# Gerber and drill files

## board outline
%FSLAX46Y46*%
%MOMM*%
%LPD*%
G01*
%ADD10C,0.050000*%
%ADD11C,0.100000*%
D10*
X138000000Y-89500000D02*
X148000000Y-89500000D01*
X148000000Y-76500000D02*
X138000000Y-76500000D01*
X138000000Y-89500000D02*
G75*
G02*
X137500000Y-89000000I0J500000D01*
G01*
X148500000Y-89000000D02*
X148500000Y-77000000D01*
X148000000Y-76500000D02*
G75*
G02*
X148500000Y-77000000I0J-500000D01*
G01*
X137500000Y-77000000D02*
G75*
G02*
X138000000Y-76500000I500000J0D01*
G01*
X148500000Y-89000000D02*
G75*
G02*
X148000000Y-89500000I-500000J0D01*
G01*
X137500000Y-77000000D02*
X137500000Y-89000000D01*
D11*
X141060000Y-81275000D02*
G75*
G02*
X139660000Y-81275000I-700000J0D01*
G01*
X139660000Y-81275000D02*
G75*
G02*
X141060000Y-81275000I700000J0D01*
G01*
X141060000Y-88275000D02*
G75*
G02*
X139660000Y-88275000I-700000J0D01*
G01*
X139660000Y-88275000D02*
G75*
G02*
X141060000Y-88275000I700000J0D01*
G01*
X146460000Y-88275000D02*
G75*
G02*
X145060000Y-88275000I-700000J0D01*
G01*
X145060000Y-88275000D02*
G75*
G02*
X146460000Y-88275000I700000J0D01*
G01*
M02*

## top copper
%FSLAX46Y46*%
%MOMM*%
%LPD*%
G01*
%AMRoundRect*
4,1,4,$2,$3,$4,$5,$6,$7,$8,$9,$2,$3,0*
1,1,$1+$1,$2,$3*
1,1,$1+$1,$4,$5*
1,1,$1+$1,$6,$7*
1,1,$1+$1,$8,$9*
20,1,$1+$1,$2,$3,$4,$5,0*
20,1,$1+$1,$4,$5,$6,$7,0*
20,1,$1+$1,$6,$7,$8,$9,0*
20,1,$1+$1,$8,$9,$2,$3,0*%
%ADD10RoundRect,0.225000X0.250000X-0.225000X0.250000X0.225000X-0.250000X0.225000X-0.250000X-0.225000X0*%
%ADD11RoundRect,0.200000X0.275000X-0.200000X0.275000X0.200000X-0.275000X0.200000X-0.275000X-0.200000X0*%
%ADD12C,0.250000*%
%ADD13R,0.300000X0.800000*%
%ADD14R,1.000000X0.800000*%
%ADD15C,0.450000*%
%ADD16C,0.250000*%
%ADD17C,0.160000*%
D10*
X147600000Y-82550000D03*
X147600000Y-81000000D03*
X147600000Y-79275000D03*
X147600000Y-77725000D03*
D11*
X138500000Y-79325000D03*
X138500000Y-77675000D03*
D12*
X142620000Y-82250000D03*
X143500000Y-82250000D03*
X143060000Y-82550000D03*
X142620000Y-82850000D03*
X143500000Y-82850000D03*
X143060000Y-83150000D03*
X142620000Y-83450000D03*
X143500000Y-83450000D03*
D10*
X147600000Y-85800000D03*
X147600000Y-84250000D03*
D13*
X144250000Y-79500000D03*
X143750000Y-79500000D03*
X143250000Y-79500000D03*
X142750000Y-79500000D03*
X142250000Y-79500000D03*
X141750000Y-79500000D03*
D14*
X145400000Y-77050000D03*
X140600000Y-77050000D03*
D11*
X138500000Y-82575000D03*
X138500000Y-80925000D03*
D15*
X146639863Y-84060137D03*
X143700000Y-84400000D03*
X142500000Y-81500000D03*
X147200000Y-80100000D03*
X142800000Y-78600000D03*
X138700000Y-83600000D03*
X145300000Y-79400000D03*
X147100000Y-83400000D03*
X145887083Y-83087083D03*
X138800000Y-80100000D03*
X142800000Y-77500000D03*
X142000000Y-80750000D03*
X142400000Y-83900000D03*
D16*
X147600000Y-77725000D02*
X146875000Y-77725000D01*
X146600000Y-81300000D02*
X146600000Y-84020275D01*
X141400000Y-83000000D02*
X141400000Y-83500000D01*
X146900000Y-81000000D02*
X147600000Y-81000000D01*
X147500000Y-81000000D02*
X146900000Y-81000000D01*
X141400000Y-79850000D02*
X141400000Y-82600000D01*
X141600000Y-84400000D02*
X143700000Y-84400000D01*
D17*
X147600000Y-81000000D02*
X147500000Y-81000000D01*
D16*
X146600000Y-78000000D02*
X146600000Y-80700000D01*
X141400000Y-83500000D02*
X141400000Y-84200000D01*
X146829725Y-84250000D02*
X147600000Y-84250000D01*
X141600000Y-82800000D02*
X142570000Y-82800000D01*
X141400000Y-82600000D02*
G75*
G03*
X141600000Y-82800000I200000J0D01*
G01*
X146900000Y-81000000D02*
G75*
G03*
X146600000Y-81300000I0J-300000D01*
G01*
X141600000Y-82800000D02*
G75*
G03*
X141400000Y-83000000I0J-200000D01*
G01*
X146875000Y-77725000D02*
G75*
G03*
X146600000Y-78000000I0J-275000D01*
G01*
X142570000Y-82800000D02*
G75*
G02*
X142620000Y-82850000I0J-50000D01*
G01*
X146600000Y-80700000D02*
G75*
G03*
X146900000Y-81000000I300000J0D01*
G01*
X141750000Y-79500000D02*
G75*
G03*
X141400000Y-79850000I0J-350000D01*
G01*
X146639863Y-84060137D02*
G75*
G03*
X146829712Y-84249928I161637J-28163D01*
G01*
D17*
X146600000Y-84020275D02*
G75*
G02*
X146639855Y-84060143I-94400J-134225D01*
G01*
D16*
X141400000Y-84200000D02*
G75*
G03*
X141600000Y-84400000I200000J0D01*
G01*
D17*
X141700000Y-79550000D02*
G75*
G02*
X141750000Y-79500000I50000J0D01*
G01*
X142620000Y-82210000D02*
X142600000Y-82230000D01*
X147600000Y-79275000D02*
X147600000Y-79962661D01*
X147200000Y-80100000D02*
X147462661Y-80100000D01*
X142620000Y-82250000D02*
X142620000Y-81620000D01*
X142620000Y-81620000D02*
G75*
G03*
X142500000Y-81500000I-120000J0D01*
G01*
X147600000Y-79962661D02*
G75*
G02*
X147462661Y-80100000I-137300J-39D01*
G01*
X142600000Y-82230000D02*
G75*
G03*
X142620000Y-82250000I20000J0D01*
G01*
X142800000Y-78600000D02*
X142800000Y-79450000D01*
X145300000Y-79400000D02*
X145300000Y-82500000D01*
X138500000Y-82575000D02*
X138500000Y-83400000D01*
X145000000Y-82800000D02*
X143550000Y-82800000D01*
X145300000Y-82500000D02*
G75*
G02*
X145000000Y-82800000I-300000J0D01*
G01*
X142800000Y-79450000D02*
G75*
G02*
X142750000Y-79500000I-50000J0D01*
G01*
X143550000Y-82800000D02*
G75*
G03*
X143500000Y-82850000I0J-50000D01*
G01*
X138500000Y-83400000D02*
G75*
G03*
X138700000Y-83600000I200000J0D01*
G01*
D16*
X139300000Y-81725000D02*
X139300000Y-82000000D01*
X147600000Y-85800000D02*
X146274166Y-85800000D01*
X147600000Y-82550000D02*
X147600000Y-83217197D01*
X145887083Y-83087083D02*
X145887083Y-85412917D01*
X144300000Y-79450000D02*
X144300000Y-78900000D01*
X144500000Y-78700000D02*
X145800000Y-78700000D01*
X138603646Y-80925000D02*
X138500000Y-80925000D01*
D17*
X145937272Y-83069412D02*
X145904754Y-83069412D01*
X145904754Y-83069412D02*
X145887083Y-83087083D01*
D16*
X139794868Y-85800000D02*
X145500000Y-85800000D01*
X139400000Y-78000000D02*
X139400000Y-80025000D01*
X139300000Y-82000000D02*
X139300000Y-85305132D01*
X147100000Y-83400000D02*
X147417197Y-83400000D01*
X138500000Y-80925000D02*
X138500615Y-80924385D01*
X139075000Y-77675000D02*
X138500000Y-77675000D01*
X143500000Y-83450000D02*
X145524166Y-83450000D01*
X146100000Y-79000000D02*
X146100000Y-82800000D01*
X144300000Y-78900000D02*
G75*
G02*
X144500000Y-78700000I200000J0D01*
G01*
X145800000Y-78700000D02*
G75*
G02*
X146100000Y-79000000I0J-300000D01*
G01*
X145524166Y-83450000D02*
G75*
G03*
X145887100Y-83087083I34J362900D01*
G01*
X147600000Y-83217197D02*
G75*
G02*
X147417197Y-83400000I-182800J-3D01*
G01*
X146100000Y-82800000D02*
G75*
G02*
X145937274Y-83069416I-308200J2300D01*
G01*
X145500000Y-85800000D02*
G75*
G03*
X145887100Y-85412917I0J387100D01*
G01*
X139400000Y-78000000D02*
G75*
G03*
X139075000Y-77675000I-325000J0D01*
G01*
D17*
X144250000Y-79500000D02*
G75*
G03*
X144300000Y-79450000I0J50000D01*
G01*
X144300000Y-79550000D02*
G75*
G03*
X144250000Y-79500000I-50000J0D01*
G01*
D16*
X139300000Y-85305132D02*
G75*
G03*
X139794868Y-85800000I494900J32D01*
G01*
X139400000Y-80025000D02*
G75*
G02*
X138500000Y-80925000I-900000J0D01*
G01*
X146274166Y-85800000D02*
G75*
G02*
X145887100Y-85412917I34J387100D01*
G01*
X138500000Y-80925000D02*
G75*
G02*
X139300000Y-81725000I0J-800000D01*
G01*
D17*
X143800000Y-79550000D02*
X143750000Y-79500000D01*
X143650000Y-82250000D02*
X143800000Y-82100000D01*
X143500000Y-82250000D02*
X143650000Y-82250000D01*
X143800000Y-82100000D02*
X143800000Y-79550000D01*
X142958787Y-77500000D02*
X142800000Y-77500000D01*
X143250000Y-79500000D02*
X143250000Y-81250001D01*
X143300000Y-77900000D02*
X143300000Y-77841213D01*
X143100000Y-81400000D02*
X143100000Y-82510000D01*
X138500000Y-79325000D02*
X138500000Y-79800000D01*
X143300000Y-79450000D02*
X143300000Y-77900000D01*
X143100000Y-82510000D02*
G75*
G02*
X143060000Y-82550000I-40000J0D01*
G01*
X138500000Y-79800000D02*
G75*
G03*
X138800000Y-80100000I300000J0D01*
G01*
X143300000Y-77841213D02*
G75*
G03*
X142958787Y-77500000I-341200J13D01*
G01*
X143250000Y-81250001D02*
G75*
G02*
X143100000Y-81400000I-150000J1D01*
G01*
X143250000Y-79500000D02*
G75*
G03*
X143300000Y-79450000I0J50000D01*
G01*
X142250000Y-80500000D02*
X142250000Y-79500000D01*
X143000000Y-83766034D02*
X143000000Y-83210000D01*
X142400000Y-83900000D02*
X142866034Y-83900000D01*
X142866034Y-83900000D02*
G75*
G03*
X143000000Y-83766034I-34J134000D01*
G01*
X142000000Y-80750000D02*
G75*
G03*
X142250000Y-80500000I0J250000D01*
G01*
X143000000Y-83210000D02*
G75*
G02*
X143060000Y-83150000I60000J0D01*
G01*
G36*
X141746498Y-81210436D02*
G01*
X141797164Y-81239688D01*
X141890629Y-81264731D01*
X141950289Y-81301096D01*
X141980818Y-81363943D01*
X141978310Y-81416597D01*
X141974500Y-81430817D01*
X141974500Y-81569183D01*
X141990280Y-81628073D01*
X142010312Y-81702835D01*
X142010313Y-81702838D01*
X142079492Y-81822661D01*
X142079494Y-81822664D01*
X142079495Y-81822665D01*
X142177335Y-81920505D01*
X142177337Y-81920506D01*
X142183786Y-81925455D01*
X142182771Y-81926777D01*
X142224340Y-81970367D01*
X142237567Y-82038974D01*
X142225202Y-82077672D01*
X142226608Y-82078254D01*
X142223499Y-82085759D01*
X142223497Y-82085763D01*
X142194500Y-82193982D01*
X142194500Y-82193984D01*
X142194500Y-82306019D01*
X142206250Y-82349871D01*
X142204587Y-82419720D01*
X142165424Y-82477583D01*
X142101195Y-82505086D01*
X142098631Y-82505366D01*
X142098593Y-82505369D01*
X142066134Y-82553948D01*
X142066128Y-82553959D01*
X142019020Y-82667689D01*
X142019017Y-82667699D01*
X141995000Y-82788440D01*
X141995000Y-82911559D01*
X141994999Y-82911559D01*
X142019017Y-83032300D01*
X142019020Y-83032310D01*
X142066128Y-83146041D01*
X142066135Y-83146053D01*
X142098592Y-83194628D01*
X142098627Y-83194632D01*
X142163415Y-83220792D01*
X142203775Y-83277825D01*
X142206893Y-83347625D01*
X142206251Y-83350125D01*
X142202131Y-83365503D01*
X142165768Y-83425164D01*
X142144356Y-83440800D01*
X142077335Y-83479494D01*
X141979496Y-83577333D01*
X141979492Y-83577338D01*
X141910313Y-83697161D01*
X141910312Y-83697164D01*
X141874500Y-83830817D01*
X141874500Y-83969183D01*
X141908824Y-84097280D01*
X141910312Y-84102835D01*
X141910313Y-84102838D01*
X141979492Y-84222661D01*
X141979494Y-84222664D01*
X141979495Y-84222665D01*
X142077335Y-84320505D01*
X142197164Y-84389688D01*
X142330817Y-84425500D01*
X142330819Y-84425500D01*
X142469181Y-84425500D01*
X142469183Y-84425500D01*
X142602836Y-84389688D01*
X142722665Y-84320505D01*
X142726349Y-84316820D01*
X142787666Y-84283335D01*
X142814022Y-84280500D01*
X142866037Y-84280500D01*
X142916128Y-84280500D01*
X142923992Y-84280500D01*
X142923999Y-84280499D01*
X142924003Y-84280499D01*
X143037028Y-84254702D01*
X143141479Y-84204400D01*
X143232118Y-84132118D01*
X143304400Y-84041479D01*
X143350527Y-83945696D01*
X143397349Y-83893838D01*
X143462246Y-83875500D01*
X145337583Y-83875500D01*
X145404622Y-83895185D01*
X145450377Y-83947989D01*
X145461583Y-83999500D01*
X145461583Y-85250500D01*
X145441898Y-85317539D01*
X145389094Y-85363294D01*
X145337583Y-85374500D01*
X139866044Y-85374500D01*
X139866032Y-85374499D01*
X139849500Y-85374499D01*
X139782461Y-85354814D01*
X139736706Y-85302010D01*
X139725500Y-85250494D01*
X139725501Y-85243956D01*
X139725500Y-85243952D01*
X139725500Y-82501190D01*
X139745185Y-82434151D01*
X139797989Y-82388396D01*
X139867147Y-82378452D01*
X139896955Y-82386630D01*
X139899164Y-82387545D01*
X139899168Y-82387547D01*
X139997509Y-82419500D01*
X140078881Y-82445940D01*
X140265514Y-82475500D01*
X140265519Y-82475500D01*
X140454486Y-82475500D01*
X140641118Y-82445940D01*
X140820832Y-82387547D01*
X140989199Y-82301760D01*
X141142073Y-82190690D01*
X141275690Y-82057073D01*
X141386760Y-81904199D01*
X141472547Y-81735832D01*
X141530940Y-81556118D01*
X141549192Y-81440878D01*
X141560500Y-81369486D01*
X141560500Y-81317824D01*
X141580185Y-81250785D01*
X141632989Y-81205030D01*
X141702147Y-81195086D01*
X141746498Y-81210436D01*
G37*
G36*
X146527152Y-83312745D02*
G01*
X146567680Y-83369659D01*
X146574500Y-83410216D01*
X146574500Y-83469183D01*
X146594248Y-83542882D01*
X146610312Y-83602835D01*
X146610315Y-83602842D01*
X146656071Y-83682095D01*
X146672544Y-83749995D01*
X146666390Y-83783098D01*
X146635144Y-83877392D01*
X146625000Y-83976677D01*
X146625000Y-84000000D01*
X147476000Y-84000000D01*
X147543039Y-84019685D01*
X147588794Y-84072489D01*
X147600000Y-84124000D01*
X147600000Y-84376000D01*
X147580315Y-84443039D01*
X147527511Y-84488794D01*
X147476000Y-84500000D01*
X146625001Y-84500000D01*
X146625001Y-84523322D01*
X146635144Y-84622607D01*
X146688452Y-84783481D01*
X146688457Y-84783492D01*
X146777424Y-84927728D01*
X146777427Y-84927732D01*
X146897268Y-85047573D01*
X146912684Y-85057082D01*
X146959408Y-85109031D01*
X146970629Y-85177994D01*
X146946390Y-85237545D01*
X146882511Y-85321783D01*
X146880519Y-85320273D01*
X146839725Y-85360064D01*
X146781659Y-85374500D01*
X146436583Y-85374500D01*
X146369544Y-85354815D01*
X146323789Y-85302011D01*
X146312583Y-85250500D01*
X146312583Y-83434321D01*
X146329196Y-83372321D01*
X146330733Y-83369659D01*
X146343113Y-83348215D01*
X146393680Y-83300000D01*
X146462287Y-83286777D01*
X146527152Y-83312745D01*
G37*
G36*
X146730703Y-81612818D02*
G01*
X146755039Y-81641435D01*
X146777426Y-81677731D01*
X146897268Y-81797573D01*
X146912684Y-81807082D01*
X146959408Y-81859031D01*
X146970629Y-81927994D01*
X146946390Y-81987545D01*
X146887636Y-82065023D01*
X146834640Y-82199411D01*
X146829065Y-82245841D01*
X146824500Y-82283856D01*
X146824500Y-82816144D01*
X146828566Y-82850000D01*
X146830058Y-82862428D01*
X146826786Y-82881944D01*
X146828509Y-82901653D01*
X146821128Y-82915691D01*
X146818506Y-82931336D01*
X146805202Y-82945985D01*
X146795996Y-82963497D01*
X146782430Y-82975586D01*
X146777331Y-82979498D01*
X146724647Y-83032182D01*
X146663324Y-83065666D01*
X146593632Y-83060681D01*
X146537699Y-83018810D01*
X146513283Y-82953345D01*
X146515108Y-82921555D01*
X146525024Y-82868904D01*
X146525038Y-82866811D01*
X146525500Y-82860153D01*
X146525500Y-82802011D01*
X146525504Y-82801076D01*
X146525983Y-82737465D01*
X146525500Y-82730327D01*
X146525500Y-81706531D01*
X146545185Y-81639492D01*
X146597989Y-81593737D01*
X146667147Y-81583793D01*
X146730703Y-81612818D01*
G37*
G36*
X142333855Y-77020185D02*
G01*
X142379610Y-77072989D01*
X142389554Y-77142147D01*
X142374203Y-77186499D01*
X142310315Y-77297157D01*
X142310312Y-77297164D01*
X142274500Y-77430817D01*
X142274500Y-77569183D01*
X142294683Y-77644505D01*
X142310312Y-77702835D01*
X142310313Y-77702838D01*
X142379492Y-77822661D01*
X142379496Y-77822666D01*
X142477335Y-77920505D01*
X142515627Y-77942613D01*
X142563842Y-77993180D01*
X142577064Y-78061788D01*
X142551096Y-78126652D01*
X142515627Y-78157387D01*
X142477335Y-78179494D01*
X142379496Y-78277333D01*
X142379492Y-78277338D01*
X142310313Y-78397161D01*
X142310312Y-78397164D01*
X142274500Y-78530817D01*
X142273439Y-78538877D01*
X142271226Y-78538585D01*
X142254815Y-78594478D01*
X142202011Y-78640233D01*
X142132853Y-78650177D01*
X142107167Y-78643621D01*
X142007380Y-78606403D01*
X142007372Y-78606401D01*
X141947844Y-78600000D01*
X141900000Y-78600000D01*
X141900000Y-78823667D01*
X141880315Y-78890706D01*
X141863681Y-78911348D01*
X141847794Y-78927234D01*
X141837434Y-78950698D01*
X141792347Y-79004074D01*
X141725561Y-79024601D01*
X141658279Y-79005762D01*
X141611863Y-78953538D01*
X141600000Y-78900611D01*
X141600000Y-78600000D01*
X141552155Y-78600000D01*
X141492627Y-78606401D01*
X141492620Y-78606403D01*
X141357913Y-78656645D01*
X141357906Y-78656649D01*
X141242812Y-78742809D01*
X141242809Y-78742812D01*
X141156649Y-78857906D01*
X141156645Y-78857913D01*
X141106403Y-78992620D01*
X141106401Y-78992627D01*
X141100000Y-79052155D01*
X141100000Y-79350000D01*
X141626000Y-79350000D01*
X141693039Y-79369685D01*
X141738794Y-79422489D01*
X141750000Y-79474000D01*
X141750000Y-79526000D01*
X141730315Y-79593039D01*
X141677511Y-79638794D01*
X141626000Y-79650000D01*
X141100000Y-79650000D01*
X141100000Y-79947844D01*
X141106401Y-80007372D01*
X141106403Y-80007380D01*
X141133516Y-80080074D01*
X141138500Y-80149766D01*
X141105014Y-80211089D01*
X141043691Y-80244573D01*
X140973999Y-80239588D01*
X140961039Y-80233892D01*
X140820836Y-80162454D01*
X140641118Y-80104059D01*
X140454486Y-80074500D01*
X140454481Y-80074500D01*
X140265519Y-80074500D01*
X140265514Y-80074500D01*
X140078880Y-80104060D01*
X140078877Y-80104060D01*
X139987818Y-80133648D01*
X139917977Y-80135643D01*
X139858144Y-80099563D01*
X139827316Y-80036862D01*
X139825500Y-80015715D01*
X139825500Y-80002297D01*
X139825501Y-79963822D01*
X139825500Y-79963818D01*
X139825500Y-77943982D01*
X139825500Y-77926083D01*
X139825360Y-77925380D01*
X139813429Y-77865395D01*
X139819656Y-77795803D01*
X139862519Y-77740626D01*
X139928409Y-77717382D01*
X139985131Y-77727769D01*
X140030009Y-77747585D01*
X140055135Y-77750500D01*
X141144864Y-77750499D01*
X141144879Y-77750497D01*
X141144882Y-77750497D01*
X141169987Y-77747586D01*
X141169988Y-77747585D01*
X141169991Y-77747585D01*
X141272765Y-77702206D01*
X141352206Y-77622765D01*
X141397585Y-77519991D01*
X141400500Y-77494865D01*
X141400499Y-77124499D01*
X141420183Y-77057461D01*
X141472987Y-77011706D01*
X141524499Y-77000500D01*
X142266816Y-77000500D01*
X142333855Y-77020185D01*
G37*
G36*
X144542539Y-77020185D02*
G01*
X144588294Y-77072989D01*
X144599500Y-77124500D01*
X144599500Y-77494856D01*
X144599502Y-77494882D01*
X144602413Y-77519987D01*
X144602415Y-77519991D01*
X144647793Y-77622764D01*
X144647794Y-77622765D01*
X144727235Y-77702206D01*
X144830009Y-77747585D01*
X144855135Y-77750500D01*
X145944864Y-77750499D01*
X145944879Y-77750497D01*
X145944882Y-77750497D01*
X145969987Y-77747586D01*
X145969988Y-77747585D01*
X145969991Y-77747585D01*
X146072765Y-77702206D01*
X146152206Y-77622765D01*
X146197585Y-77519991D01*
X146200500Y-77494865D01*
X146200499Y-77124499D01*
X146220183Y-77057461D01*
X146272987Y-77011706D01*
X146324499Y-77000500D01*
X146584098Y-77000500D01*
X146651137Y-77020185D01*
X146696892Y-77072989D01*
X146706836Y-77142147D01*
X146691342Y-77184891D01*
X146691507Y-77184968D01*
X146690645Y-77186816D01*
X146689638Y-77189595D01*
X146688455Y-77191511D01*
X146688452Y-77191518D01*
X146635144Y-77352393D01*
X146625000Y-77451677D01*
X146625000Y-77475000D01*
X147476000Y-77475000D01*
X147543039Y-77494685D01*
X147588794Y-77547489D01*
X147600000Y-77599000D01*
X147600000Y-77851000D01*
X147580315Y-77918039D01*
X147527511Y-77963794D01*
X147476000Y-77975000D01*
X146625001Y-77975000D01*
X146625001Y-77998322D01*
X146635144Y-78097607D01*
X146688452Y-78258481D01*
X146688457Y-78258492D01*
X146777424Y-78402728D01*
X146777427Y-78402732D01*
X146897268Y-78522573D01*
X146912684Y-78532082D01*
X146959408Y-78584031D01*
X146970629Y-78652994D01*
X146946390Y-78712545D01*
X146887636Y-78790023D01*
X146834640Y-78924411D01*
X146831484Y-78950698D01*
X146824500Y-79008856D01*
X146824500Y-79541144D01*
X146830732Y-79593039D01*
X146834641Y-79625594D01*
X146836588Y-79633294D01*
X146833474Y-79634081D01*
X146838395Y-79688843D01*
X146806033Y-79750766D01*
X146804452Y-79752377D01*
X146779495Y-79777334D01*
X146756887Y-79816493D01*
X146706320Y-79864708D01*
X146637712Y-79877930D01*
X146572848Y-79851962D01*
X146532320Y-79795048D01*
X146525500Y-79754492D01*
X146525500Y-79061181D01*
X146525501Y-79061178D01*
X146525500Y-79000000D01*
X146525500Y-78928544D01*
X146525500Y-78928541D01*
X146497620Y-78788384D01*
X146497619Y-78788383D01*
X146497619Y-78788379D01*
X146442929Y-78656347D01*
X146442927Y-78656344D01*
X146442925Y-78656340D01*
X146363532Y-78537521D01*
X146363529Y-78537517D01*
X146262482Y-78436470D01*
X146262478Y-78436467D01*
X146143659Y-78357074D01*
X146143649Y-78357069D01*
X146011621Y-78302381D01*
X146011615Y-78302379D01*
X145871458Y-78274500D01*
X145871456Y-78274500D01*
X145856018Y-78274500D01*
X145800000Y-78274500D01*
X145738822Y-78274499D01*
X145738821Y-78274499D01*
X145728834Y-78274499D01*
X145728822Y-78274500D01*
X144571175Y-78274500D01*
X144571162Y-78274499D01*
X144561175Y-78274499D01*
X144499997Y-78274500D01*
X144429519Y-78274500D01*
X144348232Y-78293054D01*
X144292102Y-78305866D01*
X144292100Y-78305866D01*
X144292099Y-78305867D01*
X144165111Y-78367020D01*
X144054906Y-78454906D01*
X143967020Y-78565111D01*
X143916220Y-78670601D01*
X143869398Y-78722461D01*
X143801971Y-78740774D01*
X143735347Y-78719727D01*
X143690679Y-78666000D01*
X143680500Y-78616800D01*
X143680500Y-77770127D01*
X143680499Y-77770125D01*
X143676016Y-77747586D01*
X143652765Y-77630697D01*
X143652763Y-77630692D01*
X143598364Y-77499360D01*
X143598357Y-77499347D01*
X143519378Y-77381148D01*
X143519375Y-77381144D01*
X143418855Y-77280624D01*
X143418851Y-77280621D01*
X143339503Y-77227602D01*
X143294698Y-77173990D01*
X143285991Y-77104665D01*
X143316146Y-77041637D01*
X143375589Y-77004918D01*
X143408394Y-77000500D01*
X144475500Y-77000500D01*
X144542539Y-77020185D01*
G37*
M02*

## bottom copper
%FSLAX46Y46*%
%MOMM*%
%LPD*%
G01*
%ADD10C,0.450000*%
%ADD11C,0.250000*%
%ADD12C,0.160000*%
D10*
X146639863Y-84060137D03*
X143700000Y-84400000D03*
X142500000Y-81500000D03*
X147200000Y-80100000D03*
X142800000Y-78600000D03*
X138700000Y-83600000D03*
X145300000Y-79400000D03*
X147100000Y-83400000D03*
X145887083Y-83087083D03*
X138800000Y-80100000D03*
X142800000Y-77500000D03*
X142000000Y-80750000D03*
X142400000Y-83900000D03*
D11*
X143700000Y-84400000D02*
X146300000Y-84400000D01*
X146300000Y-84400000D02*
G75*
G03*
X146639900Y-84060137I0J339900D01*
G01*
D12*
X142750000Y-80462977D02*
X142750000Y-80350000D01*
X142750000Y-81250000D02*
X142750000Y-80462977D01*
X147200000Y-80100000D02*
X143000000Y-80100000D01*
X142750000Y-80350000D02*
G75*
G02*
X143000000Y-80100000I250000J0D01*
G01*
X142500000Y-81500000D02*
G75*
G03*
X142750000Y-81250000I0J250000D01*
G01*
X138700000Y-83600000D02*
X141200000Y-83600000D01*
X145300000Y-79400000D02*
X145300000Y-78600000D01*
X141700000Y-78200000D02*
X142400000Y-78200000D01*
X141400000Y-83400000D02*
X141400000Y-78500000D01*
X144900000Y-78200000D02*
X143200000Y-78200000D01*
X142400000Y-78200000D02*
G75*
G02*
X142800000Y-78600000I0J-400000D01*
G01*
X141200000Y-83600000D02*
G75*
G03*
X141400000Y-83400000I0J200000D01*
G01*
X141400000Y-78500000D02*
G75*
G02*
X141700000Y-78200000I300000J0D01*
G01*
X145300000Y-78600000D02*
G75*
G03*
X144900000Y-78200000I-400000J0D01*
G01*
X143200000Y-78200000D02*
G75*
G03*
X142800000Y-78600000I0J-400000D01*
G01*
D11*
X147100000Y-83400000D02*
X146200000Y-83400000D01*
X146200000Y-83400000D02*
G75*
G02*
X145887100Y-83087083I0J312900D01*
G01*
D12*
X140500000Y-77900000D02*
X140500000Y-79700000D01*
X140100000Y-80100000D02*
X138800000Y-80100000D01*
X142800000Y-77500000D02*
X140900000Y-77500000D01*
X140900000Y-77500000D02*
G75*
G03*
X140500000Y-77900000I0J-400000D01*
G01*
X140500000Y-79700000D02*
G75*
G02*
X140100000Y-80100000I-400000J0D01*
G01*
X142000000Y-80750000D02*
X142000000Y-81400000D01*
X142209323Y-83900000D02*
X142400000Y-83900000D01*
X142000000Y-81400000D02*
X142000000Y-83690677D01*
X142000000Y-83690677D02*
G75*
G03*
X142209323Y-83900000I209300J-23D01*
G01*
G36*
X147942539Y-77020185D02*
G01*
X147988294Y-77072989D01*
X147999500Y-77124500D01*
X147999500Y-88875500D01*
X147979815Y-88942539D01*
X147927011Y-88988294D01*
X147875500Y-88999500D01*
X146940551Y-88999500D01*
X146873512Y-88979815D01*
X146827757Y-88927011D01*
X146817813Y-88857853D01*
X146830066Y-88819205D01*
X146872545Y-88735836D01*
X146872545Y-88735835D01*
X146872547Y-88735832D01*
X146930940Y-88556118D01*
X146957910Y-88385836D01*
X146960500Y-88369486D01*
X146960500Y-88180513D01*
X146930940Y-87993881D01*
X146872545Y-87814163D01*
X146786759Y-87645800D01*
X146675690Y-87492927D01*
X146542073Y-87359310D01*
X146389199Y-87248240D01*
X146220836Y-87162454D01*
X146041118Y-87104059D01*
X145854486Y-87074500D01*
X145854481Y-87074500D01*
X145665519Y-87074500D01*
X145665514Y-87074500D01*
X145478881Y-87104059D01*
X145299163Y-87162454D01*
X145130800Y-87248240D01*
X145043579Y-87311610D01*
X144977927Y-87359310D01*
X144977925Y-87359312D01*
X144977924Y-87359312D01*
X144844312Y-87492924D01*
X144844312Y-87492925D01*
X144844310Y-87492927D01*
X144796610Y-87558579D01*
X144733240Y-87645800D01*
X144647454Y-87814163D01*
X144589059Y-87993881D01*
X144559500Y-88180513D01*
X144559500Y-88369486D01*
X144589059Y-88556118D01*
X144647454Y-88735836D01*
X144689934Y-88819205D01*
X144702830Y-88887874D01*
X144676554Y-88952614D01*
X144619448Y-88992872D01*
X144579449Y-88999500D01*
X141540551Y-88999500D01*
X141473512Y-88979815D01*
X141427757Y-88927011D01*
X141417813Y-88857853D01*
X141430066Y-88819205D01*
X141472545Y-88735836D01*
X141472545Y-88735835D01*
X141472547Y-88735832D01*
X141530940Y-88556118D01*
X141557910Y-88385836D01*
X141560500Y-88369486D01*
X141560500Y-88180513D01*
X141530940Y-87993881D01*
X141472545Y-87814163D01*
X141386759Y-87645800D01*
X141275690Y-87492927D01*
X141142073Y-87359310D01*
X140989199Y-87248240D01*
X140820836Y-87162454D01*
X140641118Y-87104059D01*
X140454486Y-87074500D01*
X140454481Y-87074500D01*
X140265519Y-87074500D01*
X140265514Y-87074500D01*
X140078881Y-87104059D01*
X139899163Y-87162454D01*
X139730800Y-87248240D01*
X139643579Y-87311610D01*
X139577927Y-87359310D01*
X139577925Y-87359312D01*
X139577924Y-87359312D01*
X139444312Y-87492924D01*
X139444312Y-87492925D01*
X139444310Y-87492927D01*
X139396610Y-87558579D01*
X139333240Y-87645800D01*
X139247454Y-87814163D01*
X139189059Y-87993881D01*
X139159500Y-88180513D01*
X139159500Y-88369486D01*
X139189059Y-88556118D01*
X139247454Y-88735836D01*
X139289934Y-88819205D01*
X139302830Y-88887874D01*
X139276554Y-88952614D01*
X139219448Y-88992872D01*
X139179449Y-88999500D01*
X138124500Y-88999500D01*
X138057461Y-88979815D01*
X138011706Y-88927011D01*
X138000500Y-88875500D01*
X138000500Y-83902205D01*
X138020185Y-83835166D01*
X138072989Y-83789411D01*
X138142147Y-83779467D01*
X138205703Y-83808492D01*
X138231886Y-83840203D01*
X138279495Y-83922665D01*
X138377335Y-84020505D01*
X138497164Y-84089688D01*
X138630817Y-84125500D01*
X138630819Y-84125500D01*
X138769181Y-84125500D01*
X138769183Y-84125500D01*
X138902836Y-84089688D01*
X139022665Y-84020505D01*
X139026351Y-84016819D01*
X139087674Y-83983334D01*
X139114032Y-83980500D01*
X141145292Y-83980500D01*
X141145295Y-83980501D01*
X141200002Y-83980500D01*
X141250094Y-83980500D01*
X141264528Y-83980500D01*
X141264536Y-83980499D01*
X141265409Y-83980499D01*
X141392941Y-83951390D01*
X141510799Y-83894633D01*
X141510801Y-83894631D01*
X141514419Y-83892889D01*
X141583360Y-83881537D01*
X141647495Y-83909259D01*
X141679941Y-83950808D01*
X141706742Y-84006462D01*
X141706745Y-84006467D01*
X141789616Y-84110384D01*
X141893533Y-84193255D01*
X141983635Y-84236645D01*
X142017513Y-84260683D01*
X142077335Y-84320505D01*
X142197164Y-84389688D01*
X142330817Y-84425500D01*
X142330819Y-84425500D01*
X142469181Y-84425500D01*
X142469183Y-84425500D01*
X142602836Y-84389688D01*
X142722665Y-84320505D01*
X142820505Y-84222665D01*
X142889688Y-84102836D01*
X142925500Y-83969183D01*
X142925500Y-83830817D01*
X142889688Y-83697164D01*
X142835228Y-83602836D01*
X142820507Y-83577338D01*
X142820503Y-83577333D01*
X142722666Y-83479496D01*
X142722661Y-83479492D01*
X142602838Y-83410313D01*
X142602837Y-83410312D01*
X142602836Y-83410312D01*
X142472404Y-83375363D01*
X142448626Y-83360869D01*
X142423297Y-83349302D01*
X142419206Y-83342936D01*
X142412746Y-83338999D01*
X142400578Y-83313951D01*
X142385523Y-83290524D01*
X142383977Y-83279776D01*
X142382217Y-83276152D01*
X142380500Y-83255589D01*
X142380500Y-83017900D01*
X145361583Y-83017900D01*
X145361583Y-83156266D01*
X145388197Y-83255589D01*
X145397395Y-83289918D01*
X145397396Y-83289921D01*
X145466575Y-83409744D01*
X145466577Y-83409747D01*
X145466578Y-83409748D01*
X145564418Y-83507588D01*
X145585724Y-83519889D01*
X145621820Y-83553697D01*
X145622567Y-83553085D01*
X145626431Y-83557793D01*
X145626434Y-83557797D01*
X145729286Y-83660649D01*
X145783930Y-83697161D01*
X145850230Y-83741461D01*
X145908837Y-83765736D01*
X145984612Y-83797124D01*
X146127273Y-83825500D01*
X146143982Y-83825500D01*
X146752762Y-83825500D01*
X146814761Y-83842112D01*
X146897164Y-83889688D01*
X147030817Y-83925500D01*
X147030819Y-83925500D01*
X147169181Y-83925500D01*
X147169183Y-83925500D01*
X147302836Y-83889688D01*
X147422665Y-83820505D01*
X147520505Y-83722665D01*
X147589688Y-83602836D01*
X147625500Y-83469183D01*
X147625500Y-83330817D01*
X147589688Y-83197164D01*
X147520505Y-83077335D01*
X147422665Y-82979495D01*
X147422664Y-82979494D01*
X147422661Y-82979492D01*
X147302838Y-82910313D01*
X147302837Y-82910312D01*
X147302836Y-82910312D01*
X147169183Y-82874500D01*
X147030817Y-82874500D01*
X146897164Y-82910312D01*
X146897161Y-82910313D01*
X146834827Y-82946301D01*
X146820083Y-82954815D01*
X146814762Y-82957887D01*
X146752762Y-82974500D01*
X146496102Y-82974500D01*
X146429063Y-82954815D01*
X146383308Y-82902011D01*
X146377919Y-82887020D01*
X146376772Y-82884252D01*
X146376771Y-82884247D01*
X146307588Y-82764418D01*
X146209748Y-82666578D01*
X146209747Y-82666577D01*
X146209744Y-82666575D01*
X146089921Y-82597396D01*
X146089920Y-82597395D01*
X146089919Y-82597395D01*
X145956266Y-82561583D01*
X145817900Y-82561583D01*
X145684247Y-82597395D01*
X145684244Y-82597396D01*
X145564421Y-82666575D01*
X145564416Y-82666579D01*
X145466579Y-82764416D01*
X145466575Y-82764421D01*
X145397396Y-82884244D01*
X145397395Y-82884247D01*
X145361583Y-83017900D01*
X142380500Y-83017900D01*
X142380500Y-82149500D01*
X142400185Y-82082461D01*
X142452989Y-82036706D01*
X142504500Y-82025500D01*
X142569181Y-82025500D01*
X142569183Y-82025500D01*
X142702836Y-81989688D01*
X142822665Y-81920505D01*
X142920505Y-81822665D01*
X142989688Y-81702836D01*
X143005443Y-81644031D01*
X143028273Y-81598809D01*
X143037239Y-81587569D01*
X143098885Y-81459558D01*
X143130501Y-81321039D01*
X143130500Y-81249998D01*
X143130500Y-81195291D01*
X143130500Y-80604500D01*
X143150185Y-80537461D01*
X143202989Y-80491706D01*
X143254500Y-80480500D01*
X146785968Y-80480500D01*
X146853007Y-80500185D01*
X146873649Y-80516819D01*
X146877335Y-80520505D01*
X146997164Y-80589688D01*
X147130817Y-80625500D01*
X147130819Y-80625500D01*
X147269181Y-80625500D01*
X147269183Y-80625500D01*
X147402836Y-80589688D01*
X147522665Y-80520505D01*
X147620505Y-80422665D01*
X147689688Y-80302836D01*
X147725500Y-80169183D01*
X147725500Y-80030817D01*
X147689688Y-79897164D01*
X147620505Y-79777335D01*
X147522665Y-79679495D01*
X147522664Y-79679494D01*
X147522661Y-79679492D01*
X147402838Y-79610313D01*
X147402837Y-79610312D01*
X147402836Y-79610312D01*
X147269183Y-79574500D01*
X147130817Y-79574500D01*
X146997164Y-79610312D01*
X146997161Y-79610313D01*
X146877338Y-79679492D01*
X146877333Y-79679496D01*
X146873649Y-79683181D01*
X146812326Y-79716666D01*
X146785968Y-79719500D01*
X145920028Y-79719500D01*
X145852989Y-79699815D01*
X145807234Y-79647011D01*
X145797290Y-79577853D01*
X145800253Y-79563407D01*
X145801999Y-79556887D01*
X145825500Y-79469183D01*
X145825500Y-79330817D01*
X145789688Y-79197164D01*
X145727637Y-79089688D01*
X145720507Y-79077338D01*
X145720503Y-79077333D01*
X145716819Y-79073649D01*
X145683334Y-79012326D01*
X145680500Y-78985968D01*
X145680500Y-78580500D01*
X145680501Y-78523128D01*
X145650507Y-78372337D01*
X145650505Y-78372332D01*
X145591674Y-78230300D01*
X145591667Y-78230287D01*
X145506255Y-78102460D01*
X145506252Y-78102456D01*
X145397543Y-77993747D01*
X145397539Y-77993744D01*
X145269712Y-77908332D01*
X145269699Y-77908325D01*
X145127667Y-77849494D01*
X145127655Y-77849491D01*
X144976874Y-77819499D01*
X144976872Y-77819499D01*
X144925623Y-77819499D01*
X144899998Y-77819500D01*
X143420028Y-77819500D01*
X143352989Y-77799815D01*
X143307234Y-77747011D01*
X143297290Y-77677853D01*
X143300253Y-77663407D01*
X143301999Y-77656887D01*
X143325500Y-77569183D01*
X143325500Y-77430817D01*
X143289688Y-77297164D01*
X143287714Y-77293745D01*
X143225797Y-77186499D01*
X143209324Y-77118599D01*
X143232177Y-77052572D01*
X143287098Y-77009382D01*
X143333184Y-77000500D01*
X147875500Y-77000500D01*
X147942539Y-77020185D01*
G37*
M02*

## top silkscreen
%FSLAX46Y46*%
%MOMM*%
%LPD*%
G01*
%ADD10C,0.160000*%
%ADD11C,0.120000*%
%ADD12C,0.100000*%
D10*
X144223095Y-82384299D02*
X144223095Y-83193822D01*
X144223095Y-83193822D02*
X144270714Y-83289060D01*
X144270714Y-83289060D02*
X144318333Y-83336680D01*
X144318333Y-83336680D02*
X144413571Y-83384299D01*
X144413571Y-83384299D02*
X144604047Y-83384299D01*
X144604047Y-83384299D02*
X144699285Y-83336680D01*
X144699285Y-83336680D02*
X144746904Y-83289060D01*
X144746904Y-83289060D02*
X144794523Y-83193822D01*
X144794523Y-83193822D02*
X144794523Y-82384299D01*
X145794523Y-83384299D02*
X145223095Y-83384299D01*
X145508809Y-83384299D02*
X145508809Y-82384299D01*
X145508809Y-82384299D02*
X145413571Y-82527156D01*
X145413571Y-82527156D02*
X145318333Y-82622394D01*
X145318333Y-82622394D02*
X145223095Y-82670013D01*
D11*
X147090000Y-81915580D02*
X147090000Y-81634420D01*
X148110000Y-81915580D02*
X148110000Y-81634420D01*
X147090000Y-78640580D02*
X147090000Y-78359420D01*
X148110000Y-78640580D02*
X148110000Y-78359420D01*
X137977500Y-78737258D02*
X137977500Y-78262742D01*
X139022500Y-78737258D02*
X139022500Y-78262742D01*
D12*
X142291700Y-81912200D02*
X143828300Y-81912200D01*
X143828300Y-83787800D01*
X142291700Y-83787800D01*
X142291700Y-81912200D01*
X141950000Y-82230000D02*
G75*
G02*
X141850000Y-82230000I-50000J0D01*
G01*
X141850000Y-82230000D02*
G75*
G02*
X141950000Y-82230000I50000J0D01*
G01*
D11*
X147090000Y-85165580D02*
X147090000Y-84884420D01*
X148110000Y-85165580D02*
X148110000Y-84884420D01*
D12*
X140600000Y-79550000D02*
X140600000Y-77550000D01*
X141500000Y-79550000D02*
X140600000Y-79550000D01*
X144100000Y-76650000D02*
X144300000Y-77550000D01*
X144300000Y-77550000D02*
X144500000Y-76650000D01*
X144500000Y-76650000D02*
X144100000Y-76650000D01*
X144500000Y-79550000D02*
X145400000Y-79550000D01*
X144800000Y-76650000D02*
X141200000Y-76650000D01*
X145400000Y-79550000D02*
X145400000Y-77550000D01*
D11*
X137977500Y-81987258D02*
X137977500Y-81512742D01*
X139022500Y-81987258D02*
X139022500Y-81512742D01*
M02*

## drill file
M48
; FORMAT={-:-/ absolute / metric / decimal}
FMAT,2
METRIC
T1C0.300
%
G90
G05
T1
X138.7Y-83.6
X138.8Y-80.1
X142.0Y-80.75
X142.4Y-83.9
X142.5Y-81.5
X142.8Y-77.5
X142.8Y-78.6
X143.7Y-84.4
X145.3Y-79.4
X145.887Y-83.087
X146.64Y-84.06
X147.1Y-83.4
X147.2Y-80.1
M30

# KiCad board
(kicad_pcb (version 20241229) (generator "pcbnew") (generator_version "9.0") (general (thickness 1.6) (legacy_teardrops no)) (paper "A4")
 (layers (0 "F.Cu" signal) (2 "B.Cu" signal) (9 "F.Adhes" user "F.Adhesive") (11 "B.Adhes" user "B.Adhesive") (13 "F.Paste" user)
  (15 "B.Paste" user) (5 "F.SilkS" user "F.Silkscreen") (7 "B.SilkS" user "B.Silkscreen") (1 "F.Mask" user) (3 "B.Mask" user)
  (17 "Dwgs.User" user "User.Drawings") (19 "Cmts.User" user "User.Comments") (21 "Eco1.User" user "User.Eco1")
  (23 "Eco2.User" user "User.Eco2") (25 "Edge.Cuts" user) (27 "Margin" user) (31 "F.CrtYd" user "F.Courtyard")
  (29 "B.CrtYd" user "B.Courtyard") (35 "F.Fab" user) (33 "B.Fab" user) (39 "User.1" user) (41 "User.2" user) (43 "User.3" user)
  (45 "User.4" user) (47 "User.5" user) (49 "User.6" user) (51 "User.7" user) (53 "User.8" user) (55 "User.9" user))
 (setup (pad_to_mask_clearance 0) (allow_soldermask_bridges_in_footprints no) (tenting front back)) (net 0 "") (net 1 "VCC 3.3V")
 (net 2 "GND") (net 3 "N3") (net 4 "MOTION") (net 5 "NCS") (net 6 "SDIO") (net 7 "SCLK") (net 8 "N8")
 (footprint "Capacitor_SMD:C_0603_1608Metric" (layer "F.Cu") (at 147.6 81.775 90)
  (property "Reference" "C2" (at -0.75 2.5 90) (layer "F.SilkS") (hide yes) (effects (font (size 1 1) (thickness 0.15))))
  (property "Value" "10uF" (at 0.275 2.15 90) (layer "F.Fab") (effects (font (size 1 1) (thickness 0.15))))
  (fp_line (start -0.14058 -0.51) (end 0.14058 -0.51) (stroke (width 0.12) (type solid)) (layer "F.SilkS"))
  (fp_line (start -0.14058 0.51) (end 0.14058 0.51) (stroke (width 0.12) (type solid)) (layer "F.SilkS"))
  (pad "1" smd roundrect (at -0.775 0 90) (size 0.9 0.95) (layers "F.Cu" "F.Mask" "F.Paste") (roundrect_rratio 0.25) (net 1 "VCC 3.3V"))
  (pad "2" smd roundrect (at 0.775 0 90) (size 0.9 0.95) (layers "F.Cu" "F.Mask" "F.Paste") (roundrect_rratio 0.25) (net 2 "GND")))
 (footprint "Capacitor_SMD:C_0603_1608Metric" (layer "F.Cu") (at 147.6 78.5 90)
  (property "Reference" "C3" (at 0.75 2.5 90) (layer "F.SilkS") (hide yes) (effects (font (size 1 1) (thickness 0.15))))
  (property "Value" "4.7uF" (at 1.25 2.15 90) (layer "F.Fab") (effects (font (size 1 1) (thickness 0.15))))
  (fp_line (start -0.14058 -0.51) (end 0.14058 -0.51) (stroke (width 0.12) (type solid)) (layer "F.SilkS"))
  (fp_line (start -0.14058 0.51) (end 0.14058 0.51) (stroke (width 0.12) (type solid)) (layer "F.SilkS"))
  (pad "1" smd roundrect (at -0.775 0 90) (size 0.9 0.95) (layers "F.Cu" "F.Mask" "F.Paste") (roundrect_rratio 0.25) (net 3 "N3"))
  (pad "2" smd roundrect (at 0.775 0 90) (size 0.9 0.95) (layers "F.Cu" "F.Mask" "F.Paste") (roundrect_rratio 0.25) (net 2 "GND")))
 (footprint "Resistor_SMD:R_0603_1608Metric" (layer "F.Cu") (at 138.5 78.5 90)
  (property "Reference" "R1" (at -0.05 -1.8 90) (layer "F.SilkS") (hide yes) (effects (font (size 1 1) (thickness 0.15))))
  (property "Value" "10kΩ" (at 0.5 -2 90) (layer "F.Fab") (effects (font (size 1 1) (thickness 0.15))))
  (fp_line (start -0.237258 -0.5225) (end 0.237258 -0.5225) (stroke (width 0.12) (type solid)) (layer "F.SilkS"))
  (fp_line (start -0.237258 0.5225) (end 0.237258 0.5225) (stroke (width 0.12) (type solid)) (layer "F.SilkS"))
  (pad "1" smd roundrect (at -0.825 0 90) (size 0.8 0.95) (layers "F.Cu" "F.Mask" "F.Paste") (roundrect_rratio 0.25) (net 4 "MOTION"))
  (pad "2" smd roundrect (at 0.825 0 90) (size 0.8 0.95) (layers "F.Cu" "F.Mask" "F.Paste") (roundrect_rratio 0.25) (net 1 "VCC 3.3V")))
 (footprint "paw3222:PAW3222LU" (layer "F.Cu") (at 143.06 82.85)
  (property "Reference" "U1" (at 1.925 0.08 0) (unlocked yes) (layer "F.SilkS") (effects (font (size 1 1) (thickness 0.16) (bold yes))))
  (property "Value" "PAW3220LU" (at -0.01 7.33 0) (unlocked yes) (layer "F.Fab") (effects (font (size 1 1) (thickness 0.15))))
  (fp_rect (start -0.7683 -0.9378) (end 0.7683 0.9378) (stroke (width 0.1) (type default)) (fill no) (layer "F.SilkS"))
  (fp_circle (center -1.16 -0.62) (end -1.06 -0.62) (stroke (width 0) (type solid)) (fill yes) (layer "F.SilkS"))
  (fp_circle (center -2.7 -1.575) (end -2 -1.575) (stroke (width 0.1) (type default)) (fill no) (layer "Edge.Cuts"))
  (fp_circle (center -2.7 5.425) (end -2 5.425) (stroke (width 0.1) (type default)) (fill no) (layer "Edge.Cuts"))
  (fp_circle (center 2.7 5.425) (end 3.4 5.425) (stroke (width 0.1) (type default)) (fill no) (layer "Edge.Cuts"))
  (pad "A1" smd circle (at -0.44 -0.6) (size 0.25 0.25) (layers "F.Cu" "F.Mask" "F.Paste") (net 3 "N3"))
  (pad "A3" smd circle (at 0.44 -0.6) (size 0.25 0.25) (layers "F.Cu" "F.Mask" "F.Paste") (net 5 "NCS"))
  (pad "B2" smd circle (at 0 -0.3) (size 0.25 0.25) (layers "F.Cu" "F.Mask" "F.Paste") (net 4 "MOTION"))
  (pad "C1" smd circle (at -0.44 0) (size 0.25 0.25) (layers "F.Cu" "F.Mask" "F.Paste") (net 2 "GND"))
  (pad "C3" smd circle (at 0.44 0) (size 0.25 0.25) (layers "F.Cu" "F.Mask" "F.Paste") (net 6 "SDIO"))
  (pad "D2" smd circle (at 0 0.3) (size 0.25 0.25) (layers "F.Cu" "F.Mask" "F.Paste") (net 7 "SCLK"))
  (pad "E1" smd circle (at -0.44 0.6) (size 0.25 0.25) (layers "F.Cu" "F.Mask" "F.Paste") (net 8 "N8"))
  (pad "E3" smd circle (at 0.44 0.6) (size 0.25 0.25) (layers "F.Cu" "F.Mask" "F.Paste") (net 1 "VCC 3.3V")))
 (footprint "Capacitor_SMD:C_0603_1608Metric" (layer "F.Cu") (at 147.6 85.025 90)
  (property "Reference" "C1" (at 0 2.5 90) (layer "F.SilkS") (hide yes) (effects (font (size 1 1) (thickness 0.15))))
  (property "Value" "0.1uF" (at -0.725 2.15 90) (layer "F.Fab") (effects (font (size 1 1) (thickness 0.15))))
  (fp_line (start -0.14058 -0.51) (end 0.14058 -0.51) (stroke (width 0.12) (type solid)) (layer "F.SilkS"))
  (fp_line (start -0.14058 0.51) (end 0.14058 0.51) (stroke (width 0.12) (type solid)) (layer "F.SilkS"))
  (pad "1" smd roundrect (at -0.775 0 90) (size 0.9 0.95) (layers "F.Cu" "F.Mask" "F.Paste") (roundrect_rratio 0.25) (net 1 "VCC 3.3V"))
  (pad "2" smd roundrect (at 0.775 0 90) (size 0.9 0.95) (layers "F.Cu" "F.Mask" "F.Paste") (roundrect_rratio 0.25) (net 2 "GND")))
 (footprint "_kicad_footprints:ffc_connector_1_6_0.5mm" (layer "F.Cu") (at 143 71.25 180)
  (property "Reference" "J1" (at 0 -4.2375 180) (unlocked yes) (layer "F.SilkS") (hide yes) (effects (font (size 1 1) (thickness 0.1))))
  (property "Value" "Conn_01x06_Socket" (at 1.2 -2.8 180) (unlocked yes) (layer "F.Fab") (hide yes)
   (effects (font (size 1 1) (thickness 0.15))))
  (fp_line (start 2.4 -8.3) (end 2.4 -6.3) (stroke (width 0.1) (type default)) (layer "F.SilkS"))
  (fp_line (start 1.5 -8.3) (end 2.4 -8.3) (stroke (width 0.1) (type default)) (layer "F.SilkS"))
  (fp_line (start -1.1 -5.4) (end -1.3 -6.3) (stroke (width 0.1) (type default)) (layer "F.SilkS"))
  (fp_line (start -1.3 -6.3) (end -1.5 -5.4) (stroke (width 0.1) (type default)) (layer "F.SilkS"))
  (fp_line (start -1.5 -5.4) (end -1.1 -5.4) (stroke (width 0.1) (type default)) (layer "F.SilkS"))
  (fp_line (start -1.5 -8.3) (end -2.4 -8.3) (stroke (width 0.1) (type default)) (layer "F.SilkS"))
  (fp_line (start -1.8 -5.4) (end 1.8 -5.4) (stroke (width 0.1) (type default)) (layer "F.SilkS"))
  (fp_line (start -2.4 -8.3) (end -2.4 -6.3) (stroke (width 0.1) (type default)) (layer "F.SilkS"))
  (pad "1" smd rect (at -1.25 -8.25 180) (size 0.3 0.8) (layers "F.Cu" "F.Mask" "F.Paste") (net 1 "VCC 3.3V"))
  (pad "2" smd rect (at -0.75 -8.25 180) (size 0.3 0.8) (layers "F.Cu" "F.Mask" "F.Paste") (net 5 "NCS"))
  (pad "3" smd rect (at -0.25 -8.25 180) (size 0.3 0.8) (layers "F.Cu" "F.Mask" "F.Paste") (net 4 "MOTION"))
  (pad "4" smd rect (at 0.25 -8.25 180) (size 0.3 0.8) (layers "F.Cu" "F.Mask" "F.Paste") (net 6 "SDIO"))
  (pad "5" smd rect (at 0.75 -8.25 180) (size 0.3 0.8) (layers "F.Cu" "F.Mask" "F.Paste") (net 7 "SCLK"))
  (pad "6" smd rect (at 1.25 -8.25 180) (size 0.3 0.8) (layers "F.Cu" "F.Mask" "F.Paste") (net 2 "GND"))
  (pad "MP" smd rect (at -2.4 -5.8 180) (size 1 0.8) (layers "F.Cu" "F.Mask" "F.Paste"))
  (pad "MP" smd rect (at 2.4 -5.8 180) (size 1 0.8) (layers "F.Cu" "F.Mask" "F.Paste")))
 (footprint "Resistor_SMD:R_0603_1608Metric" (layer "F.Cu") (at 138.5 81.75 90)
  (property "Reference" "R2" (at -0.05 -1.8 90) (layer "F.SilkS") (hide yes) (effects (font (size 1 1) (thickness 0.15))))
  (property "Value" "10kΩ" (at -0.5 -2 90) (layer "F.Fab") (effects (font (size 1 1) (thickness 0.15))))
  (fp_line (start -0.237258 -0.5225) (end 0.237258 -0.5225) (stroke (width 0.12) (type solid)) (layer "F.SilkS"))
  (fp_line (start -0.237258 0.5225) (end 0.237258 0.5225) (stroke (width 0.12) (type solid)) (layer "F.SilkS"))
  (pad "1" smd roundrect (at -0.825 0 90) (size 0.8 0.95) (layers "F.Cu" "F.Mask" "F.Paste") (roundrect_rratio 0.25) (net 6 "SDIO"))
  (pad "2" smd roundrect (at 0.825 0 90) (size 0.8 0.95) (layers "F.Cu" "F.Mask" "F.Paste") (roundrect_rratio 0.25) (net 1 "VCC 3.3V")))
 (gr_line (start 138 89.5) (end 148 89.5) (stroke (width 0.05) (type default)) (layer "Edge.Cuts"))
 (gr_line (start 148 76.5) (end 138 76.5) (stroke (width 0.05) (type default)) (layer "Edge.Cuts"))
 (gr_arc (start 138 89.5) (mid 137.646447 89.353553) (end 137.5 89) (stroke (width 0.05) (type default)) (layer "Edge.Cuts"))
 (gr_line (start 148.5 89) (end 148.5 77) (stroke (width 0.05) (type default)) (layer "Edge.Cuts"))
 (gr_arc (start 148 76.5) (mid 148.353553 76.646447) (end 148.5 77) (stroke (width 0.05) (type default)) (layer "Edge.Cuts"))
 (gr_arc (start 137.5 77) (mid 137.646447 76.646447) (end 138 76.5) (stroke (width 0.05) (type default)) (layer "Edge.Cuts"))
 (gr_arc (start 148.5 89) (mid 148.353553 89.353553) (end 148 89.5) (stroke (width 0.05) (type default)) (layer "Edge.Cuts"))
 (gr_line (start 137.5 77) (end 137.5 89) (stroke (width 0.05) (type default)) (layer "Edge.Cuts"))
 (segment (start 147.6 77.725) (end 146.875 77.725) (width 0.25) (layer "F.Cu") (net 2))
 (segment (start 146.6 81.3) (end 146.6 84.020275) (width 0.25) (layer "F.Cu") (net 2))
 (segment (start 141.4 83) (end 141.4 83.5) (width 0.25) (layer "F.Cu") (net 2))
 (segment (start 146.9 81) (end 147.6 81) (width 0.25) (layer "F.Cu") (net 2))
 (segment (start 147.5 81) (end 146.9 81) (width 0.25) (layer "F.Cu") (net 2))
 (segment (start 141.4 79.85) (end 141.4 82.6) (width 0.25) (layer "F.Cu") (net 2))
 (segment (start 141.6 84.4) (end 143.7 84.4) (width 0.25) (layer "F.Cu") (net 2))
 (segment (start 147.6 81) (end 147.5 81) (width 0.16) (layer "F.Cu") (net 2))
 (segment (start 146.6 78) (end 146.6 80.7) (width 0.25) (layer "F.Cu") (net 2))
 (segment (start 141.4 83.5) (end 141.4 84.2) (width 0.25) (layer "F.Cu") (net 2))
 (segment (start 146.829725 84.25) (end 147.6 84.25) (width 0.25) (layer "F.Cu") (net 2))
 (segment (start 141.6 82.8) (end 142.57 82.8) (width 0.25) (layer "F.Cu") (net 2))
 (via (at 146.639863 84.060137) (size 0.45) (drill 0.3) (layers "F.Cu" "B.Cu") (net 2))
 (via (at 143.7 84.4) (size 0.45) (drill 0.3) (layers "F.Cu" "B.Cu") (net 2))
 (arc (start 141.4 82.6) (mid 141.458579 82.741421) (end 141.6 82.8) (width 0.25) (layer "F.Cu") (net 2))
 (arc (start 146.9 81) (mid 146.687868 81.087868) (end 146.6 81.3) (width 0.25) (layer "F.Cu") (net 2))
 (arc (start 141.6 82.8) (mid 141.458579 82.858579) (end 141.4 83) (width 0.25) (layer "F.Cu") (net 2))
 (arc (start 146.875 77.725) (mid 146.680546 77.805546) (end 146.6 78) (width 0.25) (layer "F.Cu") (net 2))
 (arc (start 142.57 82.8) (mid 142.605355 82.814645) (end 142.62 82.85) (width 0.25) (layer "F.Cu") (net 2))
 (arc (start 146.6 80.7) (mid 146.687868 80.912132) (end 146.9 81) (width 0.25) (layer "F.Cu") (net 2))
 (arc (start 141.75 79.5) (mid 141.502513 79.602513) (end 141.4 79.85) (width 0.25) (layer "F.Cu") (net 2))
 (arc (start 146.639863 84.060137) (mid 146.667285 84.182715) (end 146.829725 84.25) (width 0.25) (layer "F.Cu") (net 2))
 (arc (start 146.6 84.020275) (mid 146.667285 84.182715) (end 146.639863 84.060137) (width 0.16) (layer "F.Cu") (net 2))
 (arc (start 141.4 84.2) (mid 141.458579 84.341421) (end 141.6 84.4) (width 0.25) (layer "F.Cu") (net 2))
 (arc (start 141.7 79.55) (mid 141.714645 79.514645) (end 141.75 79.5) (width 0.16) (layer "F.Cu") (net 2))
 (segment (start 143.7 84.4) (end 146.3 84.4) (width 0.25) (layer "B.Cu") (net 2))
 (arc (start 146.3 84.4) (mid 146.540319 84.300456) (end 146.639863 84.060137) (width 0.25) (layer "B.Cu") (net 2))
 (segment (start 142.62 82.21) (end 142.6 82.23) (width 0.16) (layer "F.Cu") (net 3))
 (segment (start 147.6 79.275) (end 147.6 79.962661) (width 0.16) (layer "F.Cu") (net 3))
 (segment (start 147.2 80.1) (end 147.462661 80.1) (width 0.16) (layer "F.Cu") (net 3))
 (segment (start 142.62 82.25) (end 142.62 81.62) (width 0.16) (layer "F.Cu") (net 3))
 (via (at 142.5 81.5) (size 0.45) (drill 0.3) (layers "F.Cu" "B.Cu") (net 3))
 (via (at 147.2 80.1) (size 0.45) (drill 0.3) (layers "F.Cu" "B.Cu") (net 3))
 (arc (start 142.62 81.62) (mid 142.584853 81.535147) (end 142.5 81.5) (width 0.16) (layer "F.Cu") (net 3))
 (arc (start 147.6 79.962661) (mid 147.559774 80.059774) (end 147.462661 80.1) (width 0.16) (layer "F.Cu") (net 3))
 (arc (start 142.6 82.23) (mid 142.605858 82.244142) (end 142.62 82.25) (width 0.16) (layer "F.Cu") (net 3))
 (segment (start 142.75 80.462977) (end 142.75 80.35) (width 0.16) (layer "B.Cu") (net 3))
 (segment (start 142.75 81.25) (end 142.75 80.462977) (width 0.16) (layer "B.Cu") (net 3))
 (segment (start 147.2 80.1) (end 143 80.1) (width 0.16) (layer "B.Cu") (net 3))
 (arc (start 142.75 80.35) (mid 142.823223 80.173223) (end 143 80.1) (width 0.16) (layer "B.Cu") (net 3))
 (arc (start 142.5 81.5) (mid 142.676777 81.426777) (end 142.75 81.25) (width 0.16) (layer "B.Cu") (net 3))
 (segment (start 142.8 78.6) (end 142.8 79.45) (width 0.16) (layer "F.Cu") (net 6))
 (segment (start 145.3 79.4) (end 145.3 82.5) (width 0.16) (layer "F.Cu") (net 6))
 (segment (start 138.5 82.575) (end 138.5 83.4) (width 0.16) (layer "F.Cu") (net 6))
 (segment (start 145 82.8) (end 143.55 82.8) (width 0.16) (layer "F.Cu") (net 6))
 (via (at 142.8 78.6) (size 0.45) (drill 0.3) (layers "F.Cu" "B.Cu") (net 6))
 (via (at 138.7 83.6) (size 0.45) (drill 0.3) (layers "F.Cu" "B.Cu") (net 6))
 (via (at 145.3 79.4) (size 0.45) (drill 0.3) (layers "F.Cu" "B.Cu") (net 6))
 (arc (start 145.3 82.5) (mid 145.212132 82.712132) (end 145 82.8) (width 0.16) (layer "F.Cu") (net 6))
 (arc (start 142.8 79.45) (mid 142.785355 79.485355) (end 142.75 79.5) (width 0.16) (layer "F.Cu") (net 6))
 (arc (start 143.55 82.8) (mid 143.514645 82.814645) (end 143.5 82.85) (width 0.16) (layer "F.Cu") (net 6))
 (arc (start 138.5 83.4) (mid 138.558579 83.541421) (end 138.7 83.6) (width 0.16) (layer "F.Cu") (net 6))
 (segment (start 138.7 83.6) (end 141.2 83.6) (width 0.16) (layer "B.Cu") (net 6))
 (segment (start 145.3 79.4) (end 145.3 78.6) (width 0.16) (layer "B.Cu") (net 6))
 (segment (start 141.7 78.2) (end 142.4 78.2) (width 0.16) (layer "B.Cu") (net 6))
 (segment (start 141.4 83.4) (end 141.4 78.5) (width 0.16) (layer "B.Cu") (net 6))
 (segment (start 144.9 78.2) (end 143.2 78.2) (width 0.16) (layer "B.Cu") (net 6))
 (arc (start 142.4 78.2) (mid 142.682843 78.317157) (end 142.8 78.6) (width 0.16) (layer "B.Cu") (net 6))
 (arc (start 141.2 83.6) (mid 141.341421 83.541421) (end 141.4 83.4) (width 0.16) (layer "B.Cu") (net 6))
 (arc (start 141.4 78.5) (mid 141.487868 78.287868) (end 141.7 78.2) (width 0.16) (layer "B.Cu") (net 6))
 (arc (start 145.3 78.6) (mid 145.182843 78.317157) (end 144.9 78.2) (width 0.16) (layer "B.Cu") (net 6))
 (arc (start 143.2 78.2) (mid 142.917157 78.317157) (end 142.8 78.6) (width 0.16) (layer "B.Cu") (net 6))
 (segment (start 139.3 81.725) (end 139.3 82) (width 0.25) (layer "F.Cu") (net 1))
 (segment (start 147.6 85.8) (end 146.274166 85.8) (width 0.25) (layer "F.Cu") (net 1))
 (segment (start 147.6 82.55) (end 147.6 83.217197) (width 0.25) (layer "F.Cu") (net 1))
 (segment (start 145.887083 83.087083) (end 145.887083 85.412917) (width 0.25) (layer "F.Cu") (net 1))
 (segment (start 144.3 79.45) (end 144.3 78.9) (width 0.25) (layer "F.Cu") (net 1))
 (segment (start 144.5 78.7) (end 145.8 78.7) (width 0.25) (layer "F.Cu") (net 1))
 (segment (start 138.603646 80.925) (end 138.5 80.925) (width 0.25) (layer "F.Cu") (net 1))
 (segment (start 145.937272 83.069412) (end 145.904754 83.069412) (width 0.16) (layer "F.Cu") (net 1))
 (segment (start 145.904754 83.069412) (end 145.887083 83.087083) (width 0.16) (layer "F.Cu") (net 1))
 (segment (start 139.794868 85.8) (end 145.5 85.8) (width 0.25) (layer "F.Cu") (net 1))
 (segment (start 139.4 78) (end 139.4 80.025) (width 0.25) (layer "F.Cu") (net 1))
 (segment (start 139.3 82) (end 139.3 85.305132) (width 0.25) (layer "F.Cu") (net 1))
 (segment (start 147.1 83.4) (end 147.417197 83.4) (width 0.25) (layer "F.Cu") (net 1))
 (segment (start 138.5 80.925) (end 138.500615 80.924385) (width 0.25) (layer "F.Cu") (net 1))
 (segment (start 139.075 77.675) (end 138.5 77.675) (width 0.25) (layer "F.Cu") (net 1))
 (segment (start 143.5 83.45) (end 145.524166 83.45) (width 0.25) (layer "F.Cu") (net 1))
 (segment (start 146.1 79) (end 146.1 82.8) (width 0.25) (layer "F.Cu") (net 1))
 (via (at 147.1 83.4) (size 0.45) (drill 0.3) (layers "F.Cu" "B.Cu") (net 1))
 (via (at 145.887083 83.087083) (size 0.45) (drill 0.3) (layers "F.Cu" "B.Cu") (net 1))
 (arc (start 144.3 78.9) (mid 144.358579 78.758579) (end 144.5 78.7) (width 0.25) (layer "F.Cu") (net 1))
 (arc (start 145.8 78.7) (mid 146.012132 78.787868) (end 146.1 79) (width 0.25) (layer "F.Cu") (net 1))
 (arc (start 145.524166 83.45) (mid 145.780787 83.343704) (end 145.887083 83.087083) (width 0.25) (layer "F.Cu") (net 1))
 (arc (start 147.6 83.217197) (mid 147.546458 83.346458) (end 147.417197 83.4) (width 0.25) (layer "F.Cu") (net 1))
 (arc (start 146.1 82.8) (mid 146.055792 82.95675) (end 145.937272 83.069412) (width 0.25) (layer "F.Cu") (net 1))
 (arc (start 145.5 85.8) (mid 145.773709 85.686626) (end 145.887083 85.412917) (width 0.25) (layer "F.Cu") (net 1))
 (arc (start 139.4 78) (mid 139.30481 77.77019) (end 139.075 77.675) (width 0.25) (layer "F.Cu") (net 1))
 (arc (start 144.25 79.5) (mid 144.285355 79.485355) (end 144.3 79.45) (width 0.16) (layer "F.Cu") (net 1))
 (arc (start 144.3 79.55) (mid 144.285355 79.514645) (end 144.25 79.5) (width 0.16) (layer "F.Cu") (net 1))
 (arc (start 139.3 85.305132) (mid 139.444943 85.655057) (end 139.794868 85.8) (width 0.25) (layer "F.Cu") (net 1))
 (arc (start 139.4 80.025) (mid 139.136396 80.661396) (end 138.5 80.925) (width 0.25) (layer "F.Cu") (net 1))
 (arc (start 146.274166 85.8) (mid 146.000457 85.686626) (end 145.887083 85.412917) (width 0.25) (layer "F.Cu") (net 1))
 (arc (start 138.5 80.925) (mid 139.065685 81.159315) (end 139.3 81.725) (width 0.25) (layer "F.Cu") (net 1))
 (segment (start 147.1 83.4) (end 146.2 83.4) (width 0.25) (layer "B.Cu") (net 1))
 (arc (start 146.2 83.4) (mid 145.978734 83.308349) (end 145.887083 83.087083) (width 0.25) (layer "B.Cu") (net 1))
 (segment (start 143.8 79.55) (end 143.75 79.5) (width 0.16) (layer "F.Cu") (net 5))
 (segment (start 143.65 82.25) (end 143.8 82.1) (width 0.16) (layer "F.Cu") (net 5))
 (segment (start 143.5 82.25) (end 143.65 82.25) (width 0.16) (layer "F.Cu") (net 5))
 (segment (start 143.8 82.1) (end 143.8 79.55) (width 0.16) (layer "F.Cu") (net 5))
 (segment (start 142.958787 77.5) (end 142.8 77.5) (width 0.16) (layer "F.Cu") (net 4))
 (segment (start 143.25 79.5) (end 143.25 81.250001) (width 0.16) (layer "F.Cu") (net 4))
 (segment (start 143.3 77.9) (end 143.3 77.841213) (width 0.16) (layer "F.Cu") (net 4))
 (segment (start 143.1 81.4) (end 143.1 82.51) (width 0.16) (layer "F.Cu") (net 4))
 (segment (start 138.5 79.325) (end 138.5 79.8) (width 0.16) (layer "F.Cu") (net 4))
 (segment (start 143.3 79.45) (end 143.3 77.9) (width 0.16) (layer "F.Cu") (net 4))
 (via (at 138.8 80.1) (size 0.45) (drill 0.3) (layers "F.Cu" "B.Cu") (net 4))
 (via (at 142.8 77.5) (size 0.45) (drill 0.3) (layers "F.Cu" "B.Cu") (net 4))
 (arc (start 143.1 82.51) (mid 143.088284 82.538284) (end 143.06 82.55) (width 0.16) (layer "F.Cu") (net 4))
 (arc (start 138.5 79.8) (mid 138.587868 80.012132) (end 138.8 80.1) (width 0.16) (layer "F.Cu") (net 4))
 (arc (start 143.3 77.841213) (mid 143.200061 77.599939) (end 142.958787 77.5) (width 0.16) (layer "F.Cu") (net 4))
 (arc (start 143.25 81.250001) (mid 143.206066 81.356066) (end 143.1 81.4) (width 0.16) (layer "F.Cu") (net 4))
 (arc (start 143.25 79.5) (mid 143.285355 79.485355) (end 143.3 79.45) (width 0.16) (layer "F.Cu") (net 4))
 (segment (start 140.5 77.9) (end 140.5 79.7) (width 0.16) (layer "B.Cu") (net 4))
 (segment (start 140.1 80.1) (end 138.8 80.1) (width 0.16) (layer "B.Cu") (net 4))
 (segment (start 142.8 77.5) (end 140.9 77.5) (width 0.16) (layer "B.Cu") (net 4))
 (arc (start 140.9 77.5) (mid 140.617157 77.617157) (end 140.5 77.9) (width 0.16) (layer "B.Cu") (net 4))
 (arc (start 140.5 79.7) (mid 140.382843 79.982843) (end 140.1 80.1) (width 0.16) (layer "B.Cu") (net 4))
 (segment (start 142.25 80.5) (end 142.25 79.5) (width 0.16) (layer "F.Cu") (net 7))
 (segment (start 143 83.766034) (end 143 83.21) (width 0.16) (layer "F.Cu") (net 7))
 (segment (start 142.4 83.9) (end 142.866034 83.9) (width 0.16) (layer "F.Cu") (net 7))
 (via (at 142 80.75) (size 0.45) (drill 0.3) (layers "F.Cu" "B.Cu") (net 7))
 (via (at 142.4 83.9) (size 0.45) (drill 0.3) (layers "F.Cu" "B.Cu") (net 7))
 (arc (start 142.866034 83.9) (mid 142.960762 83.860762) (end 143 83.766034) (width 0.16) (layer "F.Cu") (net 7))
 (arc (start 142 80.75) (mid 142.176777 80.676777) (end 142.25 80.5) (width 0.16) (layer "F.Cu") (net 7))
 (arc (start 143 83.21) (mid 143.017574 83.167574) (end 143.06 83.15) (width 0.16) (layer "F.Cu") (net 7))
 (segment (start 142 80.75) (end 142 81.4) (width 0.16) (layer "B.Cu") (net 7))
 (segment (start 142.209323 83.9) (end 142.4 83.9) (width 0.16) (layer "B.Cu") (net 7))
 (segment (start 142 81.4) (end 142 83.690677) (width 0.16) (layer "B.Cu") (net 7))
 (arc (start 142 83.690677) (mid 142.061309 83.838691) (end 142.209323 83.9) (width 0.16) (layer "B.Cu") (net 7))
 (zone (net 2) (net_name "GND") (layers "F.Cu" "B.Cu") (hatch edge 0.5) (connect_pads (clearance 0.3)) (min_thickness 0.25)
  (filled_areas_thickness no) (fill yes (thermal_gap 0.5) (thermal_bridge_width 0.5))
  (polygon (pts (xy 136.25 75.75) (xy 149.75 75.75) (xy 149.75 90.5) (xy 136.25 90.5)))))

